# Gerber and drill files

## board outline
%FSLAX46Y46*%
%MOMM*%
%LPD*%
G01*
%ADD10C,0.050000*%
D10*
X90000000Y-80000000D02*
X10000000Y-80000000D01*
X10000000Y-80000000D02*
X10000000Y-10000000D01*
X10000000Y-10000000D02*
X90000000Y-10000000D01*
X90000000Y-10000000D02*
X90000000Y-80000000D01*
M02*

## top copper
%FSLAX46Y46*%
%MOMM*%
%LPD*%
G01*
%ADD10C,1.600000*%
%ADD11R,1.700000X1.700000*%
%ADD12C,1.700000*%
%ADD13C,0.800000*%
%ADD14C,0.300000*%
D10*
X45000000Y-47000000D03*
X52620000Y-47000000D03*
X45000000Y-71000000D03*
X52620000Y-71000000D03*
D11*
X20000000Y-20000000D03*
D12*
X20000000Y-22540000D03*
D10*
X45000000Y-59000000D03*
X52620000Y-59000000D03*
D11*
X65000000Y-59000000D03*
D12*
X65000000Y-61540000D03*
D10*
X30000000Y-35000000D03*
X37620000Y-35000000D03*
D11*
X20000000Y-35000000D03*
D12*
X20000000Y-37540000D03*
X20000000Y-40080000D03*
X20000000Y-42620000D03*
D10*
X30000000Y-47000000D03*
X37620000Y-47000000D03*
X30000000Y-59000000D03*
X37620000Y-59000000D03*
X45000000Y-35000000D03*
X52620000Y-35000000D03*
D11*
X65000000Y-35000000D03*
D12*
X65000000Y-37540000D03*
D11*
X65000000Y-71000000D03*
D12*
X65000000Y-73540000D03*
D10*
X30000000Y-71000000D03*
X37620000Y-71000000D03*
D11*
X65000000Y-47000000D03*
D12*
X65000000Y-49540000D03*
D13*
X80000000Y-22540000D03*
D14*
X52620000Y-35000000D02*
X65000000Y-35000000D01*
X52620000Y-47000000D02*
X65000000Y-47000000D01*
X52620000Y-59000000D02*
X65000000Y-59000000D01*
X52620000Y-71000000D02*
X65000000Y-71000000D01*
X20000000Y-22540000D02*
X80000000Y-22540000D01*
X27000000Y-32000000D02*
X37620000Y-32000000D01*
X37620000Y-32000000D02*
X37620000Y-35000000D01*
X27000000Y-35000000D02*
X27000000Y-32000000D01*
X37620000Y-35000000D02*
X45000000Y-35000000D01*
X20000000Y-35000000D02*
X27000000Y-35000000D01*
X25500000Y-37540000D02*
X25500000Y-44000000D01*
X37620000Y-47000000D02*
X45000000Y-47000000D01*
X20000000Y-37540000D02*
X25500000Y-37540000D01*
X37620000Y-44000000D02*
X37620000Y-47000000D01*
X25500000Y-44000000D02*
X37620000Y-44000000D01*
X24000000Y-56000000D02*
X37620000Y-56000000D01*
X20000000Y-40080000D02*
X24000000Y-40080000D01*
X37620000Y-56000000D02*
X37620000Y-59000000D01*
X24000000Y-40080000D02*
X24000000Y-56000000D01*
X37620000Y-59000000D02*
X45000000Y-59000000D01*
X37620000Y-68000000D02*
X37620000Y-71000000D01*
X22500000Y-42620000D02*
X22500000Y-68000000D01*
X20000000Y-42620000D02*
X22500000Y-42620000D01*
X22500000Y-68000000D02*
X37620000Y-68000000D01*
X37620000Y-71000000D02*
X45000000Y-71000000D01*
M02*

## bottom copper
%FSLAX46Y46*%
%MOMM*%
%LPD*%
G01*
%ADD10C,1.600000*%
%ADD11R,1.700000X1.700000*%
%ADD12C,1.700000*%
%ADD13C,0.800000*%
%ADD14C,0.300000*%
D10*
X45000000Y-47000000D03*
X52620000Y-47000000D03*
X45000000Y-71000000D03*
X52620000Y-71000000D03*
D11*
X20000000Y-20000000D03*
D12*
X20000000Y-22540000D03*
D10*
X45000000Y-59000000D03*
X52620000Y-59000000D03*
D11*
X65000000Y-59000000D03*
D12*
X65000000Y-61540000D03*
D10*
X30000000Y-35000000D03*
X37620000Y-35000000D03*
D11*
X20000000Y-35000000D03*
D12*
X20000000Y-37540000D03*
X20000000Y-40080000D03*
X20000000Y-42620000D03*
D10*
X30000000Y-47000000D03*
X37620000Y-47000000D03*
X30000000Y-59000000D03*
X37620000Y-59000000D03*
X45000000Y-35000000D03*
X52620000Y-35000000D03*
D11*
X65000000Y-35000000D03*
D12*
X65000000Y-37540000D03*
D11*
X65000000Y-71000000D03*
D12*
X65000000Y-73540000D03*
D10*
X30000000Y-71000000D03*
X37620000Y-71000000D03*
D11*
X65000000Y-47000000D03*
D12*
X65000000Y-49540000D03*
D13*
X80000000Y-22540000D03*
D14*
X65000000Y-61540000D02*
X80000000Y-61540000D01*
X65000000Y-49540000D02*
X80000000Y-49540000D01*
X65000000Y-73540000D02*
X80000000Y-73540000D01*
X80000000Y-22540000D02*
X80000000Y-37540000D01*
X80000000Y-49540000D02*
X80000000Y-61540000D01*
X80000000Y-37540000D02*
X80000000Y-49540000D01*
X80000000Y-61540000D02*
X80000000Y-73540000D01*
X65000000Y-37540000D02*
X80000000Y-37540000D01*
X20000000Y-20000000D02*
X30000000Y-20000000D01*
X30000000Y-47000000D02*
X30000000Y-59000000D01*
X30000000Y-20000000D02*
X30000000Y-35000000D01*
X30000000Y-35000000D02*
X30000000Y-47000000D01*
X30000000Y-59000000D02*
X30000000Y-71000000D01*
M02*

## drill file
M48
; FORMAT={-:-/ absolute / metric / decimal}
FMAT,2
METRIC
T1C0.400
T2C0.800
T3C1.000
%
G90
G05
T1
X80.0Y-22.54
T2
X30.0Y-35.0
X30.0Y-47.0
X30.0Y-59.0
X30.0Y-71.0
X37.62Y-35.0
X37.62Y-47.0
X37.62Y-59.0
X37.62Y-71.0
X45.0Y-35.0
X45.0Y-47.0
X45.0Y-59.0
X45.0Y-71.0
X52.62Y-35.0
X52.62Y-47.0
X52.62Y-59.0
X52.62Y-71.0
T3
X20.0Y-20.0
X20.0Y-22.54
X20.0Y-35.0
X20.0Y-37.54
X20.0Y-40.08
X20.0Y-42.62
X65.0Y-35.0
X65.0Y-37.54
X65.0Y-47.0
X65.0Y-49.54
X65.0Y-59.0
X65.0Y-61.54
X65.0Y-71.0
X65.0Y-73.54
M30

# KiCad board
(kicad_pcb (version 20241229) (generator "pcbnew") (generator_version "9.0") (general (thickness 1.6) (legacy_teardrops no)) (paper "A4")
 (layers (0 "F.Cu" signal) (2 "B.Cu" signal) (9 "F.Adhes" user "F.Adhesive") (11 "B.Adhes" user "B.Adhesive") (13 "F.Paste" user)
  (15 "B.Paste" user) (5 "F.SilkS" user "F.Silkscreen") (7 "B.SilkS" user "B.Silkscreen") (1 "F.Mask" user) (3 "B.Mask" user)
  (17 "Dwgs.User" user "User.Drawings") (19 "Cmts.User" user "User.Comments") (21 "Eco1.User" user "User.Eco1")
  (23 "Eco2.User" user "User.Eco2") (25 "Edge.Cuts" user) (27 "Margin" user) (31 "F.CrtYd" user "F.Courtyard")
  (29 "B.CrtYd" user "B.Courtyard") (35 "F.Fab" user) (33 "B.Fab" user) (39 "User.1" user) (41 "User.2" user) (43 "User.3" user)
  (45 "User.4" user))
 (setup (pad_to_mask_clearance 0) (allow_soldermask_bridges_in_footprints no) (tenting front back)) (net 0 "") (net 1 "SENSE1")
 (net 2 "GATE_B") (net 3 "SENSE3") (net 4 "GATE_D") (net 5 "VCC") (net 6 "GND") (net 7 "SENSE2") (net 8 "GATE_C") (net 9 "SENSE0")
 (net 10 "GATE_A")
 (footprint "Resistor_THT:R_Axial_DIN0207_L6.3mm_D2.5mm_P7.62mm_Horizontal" (layer "F.Cu") (at 45 47)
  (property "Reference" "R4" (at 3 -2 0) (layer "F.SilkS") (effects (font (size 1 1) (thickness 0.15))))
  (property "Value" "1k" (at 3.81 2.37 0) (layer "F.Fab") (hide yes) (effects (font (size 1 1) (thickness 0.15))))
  (pad "1" thru_hole circle (at 0 0) (size 1.6 1.6) (drill 0.8) (layers "*.Cu" "*.Mask") (remove_unused_layers no) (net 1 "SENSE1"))
  (pad "2" thru_hole circle (at 7.62 0) (size 1.6 1.6) (drill 0.8) (layers "*.Cu" "*.Mask") (remove_unused_layers no) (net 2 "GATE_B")))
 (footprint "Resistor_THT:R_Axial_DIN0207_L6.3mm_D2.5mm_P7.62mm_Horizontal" (layer "F.Cu") (at 45 71)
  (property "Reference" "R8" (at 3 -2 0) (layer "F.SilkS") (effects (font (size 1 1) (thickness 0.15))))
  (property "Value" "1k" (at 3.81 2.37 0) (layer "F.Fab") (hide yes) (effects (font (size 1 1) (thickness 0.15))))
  (pad "1" thru_hole circle (at 0 0) (size 1.6 1.6) (drill 0.8) (layers "*.Cu" "*.Mask") (remove_unused_layers no) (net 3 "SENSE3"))
  (pad "2" thru_hole circle (at 7.62 0) (size 1.6 1.6) (drill 0.8) (layers "*.Cu" "*.Mask") (remove_unused_layers no) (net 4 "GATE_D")))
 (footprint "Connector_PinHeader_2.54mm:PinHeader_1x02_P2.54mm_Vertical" (layer "F.Cu") (at 20 20)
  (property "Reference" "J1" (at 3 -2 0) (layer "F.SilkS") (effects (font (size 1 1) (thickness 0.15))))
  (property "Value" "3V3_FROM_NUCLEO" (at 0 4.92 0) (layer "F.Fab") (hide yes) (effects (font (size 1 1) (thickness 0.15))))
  (pad "1" thru_hole rect (at 0 0) (size 1.7 1.7) (drill 1) (layers "*.Cu" "*.Mask") (remove_unused_layers no) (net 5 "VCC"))
  (pad "2" thru_hole circle (at 0 2.54) (size 1.7 1.7) (drill 1) (layers "*.Cu" "*.Mask") (remove_unused_layers no) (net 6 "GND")))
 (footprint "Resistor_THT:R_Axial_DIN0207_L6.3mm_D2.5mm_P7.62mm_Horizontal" (layer "F.Cu") (at 45 59)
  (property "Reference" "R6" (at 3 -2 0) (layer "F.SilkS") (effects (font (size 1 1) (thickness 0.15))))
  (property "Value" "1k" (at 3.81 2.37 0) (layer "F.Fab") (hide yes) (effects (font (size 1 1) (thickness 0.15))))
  (pad "1" thru_hole circle (at 0 0) (size 1.6 1.6) (drill 0.8) (layers "*.Cu" "*.Mask") (remove_unused_layers no) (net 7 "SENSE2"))
  (pad "2" thru_hole circle (at 7.62 0) (size 1.6 1.6) (drill 0.8) (layers "*.Cu" "*.Mask") (remove_unused_layers no) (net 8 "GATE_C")))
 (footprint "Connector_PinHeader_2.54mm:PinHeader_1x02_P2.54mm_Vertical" (layer "F.Cu") (at 65 59)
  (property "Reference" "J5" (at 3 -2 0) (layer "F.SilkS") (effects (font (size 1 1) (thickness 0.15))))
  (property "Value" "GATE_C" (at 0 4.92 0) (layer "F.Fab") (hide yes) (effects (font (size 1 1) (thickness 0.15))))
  (pad "1" thru_hole rect (at 0 0) (size 1.7 1.7) (drill 1) (layers "*.Cu" "*.Mask") (remove_unused_layers no) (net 8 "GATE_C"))
  (pad "2" thru_hole circle (at 0 2.54) (size 1.7 1.7) (drill 1) (layers "*.Cu" "*.Mask") (remove_unused_layers no) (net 6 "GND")))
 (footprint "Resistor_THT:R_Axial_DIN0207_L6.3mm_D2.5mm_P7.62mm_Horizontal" (layer "F.Cu") (at 30 35)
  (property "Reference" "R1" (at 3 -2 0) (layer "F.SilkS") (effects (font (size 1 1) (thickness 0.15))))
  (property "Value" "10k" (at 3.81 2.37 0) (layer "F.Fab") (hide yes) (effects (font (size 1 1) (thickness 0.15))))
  (pad "1" thru_hole circle (at 0 0) (size 1.6 1.6) (drill 0.8) (layers "*.Cu" "*.Mask") (remove_unused_layers no) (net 5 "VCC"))
  (pad "2" thru_hole circle (at 7.62 0) (size 1.6 1.6) (drill 0.8) (layers "*.Cu" "*.Mask") (remove_unused_layers no) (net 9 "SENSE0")))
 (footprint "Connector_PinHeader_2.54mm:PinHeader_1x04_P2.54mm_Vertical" (layer "F.Cu") (at 20 35)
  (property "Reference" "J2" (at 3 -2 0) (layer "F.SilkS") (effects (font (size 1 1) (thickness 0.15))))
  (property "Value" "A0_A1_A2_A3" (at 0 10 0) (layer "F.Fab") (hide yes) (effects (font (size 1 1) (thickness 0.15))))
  (pad "1" thru_hole rect (at 0 0) (size 1.7 1.7) (drill 1) (layers "*.Cu" "*.Mask") (remove_unused_layers no) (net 9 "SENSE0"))
  (pad "2" thru_hole circle (at 0 2.54) (size 1.7 1.7) (drill 1) (layers "*.Cu" "*.Mask") (remove_unused_layers no) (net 1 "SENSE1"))
  (pad "3" thru_hole circle (at 0 5.08) (size 1.7 1.7) (drill 1) (layers "*.Cu" "*.Mask") (remove_unused_layers no) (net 7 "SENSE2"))
  (pad "4" thru_hole circle (at 0 7.62) (size 1.7 1.7) (drill 1) (layers "*.Cu" "*.Mask") (remove_unused_layers no) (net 3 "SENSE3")))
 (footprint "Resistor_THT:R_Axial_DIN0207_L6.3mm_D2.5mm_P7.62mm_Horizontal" (layer "F.Cu") (at 30 47)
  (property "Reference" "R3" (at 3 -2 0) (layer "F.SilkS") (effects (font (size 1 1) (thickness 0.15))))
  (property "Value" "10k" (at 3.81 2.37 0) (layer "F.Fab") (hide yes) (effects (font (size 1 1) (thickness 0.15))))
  (pad "1" thru_hole circle (at 0 0) (size 1.6 1.6) (drill 0.8) (layers "*.Cu" "*.Mask") (remove_unused_layers no) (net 5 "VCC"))
  (pad "2" thru_hole circle (at 7.62 0) (size 1.6 1.6) (drill 0.8) (layers "*.Cu" "*.Mask") (remove_unused_layers no) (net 1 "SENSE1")))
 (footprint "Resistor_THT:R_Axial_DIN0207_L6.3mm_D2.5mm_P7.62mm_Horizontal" (layer "F.Cu") (at 30 59)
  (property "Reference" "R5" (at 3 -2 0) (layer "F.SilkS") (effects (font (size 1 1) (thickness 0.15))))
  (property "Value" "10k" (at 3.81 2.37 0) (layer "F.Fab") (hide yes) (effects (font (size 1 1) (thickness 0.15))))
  (pad "1" thru_hole circle (at 0 0) (size 1.6 1.6) (drill 0.8) (layers "*.Cu" "*.Mask") (remove_unused_layers no) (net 5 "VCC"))
  (pad "2" thru_hole circle (at 7.62 0) (size 1.6 1.6) (drill 0.8) (layers "*.Cu" "*.Mask") (remove_unused_layers no) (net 7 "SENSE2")))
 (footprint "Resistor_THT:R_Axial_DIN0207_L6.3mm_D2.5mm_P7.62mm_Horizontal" (layer "F.Cu") (at 45 35)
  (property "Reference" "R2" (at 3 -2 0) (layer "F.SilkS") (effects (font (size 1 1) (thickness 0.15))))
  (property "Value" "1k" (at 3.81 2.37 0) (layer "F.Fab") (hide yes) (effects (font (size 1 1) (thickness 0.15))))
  (pad "1" thru_hole circle (at 0 0) (size 1.6 1.6) (drill 0.8) (layers "*.Cu" "*.Mask") (remove_unused_layers no) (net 9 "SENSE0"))
  (pad "2" thru_hole circle (at 7.62 0) (size 1.6 1.6) (drill 0.8) (layers "*.Cu" "*.Mask") (remove_unused_layers no) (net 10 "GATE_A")))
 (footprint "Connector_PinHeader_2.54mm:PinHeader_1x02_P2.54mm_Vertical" (layer "F.Cu") (at 65 35)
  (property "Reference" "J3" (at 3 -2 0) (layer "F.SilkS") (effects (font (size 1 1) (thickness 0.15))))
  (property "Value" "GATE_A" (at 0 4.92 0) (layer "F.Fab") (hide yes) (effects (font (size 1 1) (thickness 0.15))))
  (pad "1" thru_hole rect (at 0 0) (size 1.7 1.7) (drill 1) (layers "*.Cu" "*.Mask") (remove_unused_layers no) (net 10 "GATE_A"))
  (pad "2" thru_hole circle (at 0 2.54) (size 1.7 1.7) (drill 1) (layers "*.Cu" "*.Mask") (remove_unused_layers no) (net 6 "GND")))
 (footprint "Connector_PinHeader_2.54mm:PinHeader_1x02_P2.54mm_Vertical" (layer "F.Cu") (at 65 71)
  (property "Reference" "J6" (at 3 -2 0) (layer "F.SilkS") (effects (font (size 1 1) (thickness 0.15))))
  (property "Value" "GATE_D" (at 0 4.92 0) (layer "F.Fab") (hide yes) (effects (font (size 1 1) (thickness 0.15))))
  (pad "1" thru_hole rect (at 0 0) (size 1.7 1.7) (drill 1) (layers "*.Cu" "*.Mask") (remove_unused_layers no) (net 4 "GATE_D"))
  (pad "2" thru_hole circle (at 0 2.54) (size 1.7 1.7) (drill 1) (layers "*.Cu" "*.Mask") (remove_unused_layers no) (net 6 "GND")))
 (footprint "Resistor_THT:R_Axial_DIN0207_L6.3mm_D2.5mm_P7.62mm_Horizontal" (layer "F.Cu") (at 30 71)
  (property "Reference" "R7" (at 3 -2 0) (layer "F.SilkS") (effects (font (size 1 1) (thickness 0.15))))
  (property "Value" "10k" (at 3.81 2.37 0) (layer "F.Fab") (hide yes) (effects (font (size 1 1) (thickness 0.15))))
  (pad "1" thru_hole circle (at 0 0) (size 1.6 1.6) (drill 0.8) (layers "*.Cu" "*.Mask") (remove_unused_layers no) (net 5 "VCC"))
  (pad "2" thru_hole circle (at 7.62 0) (size 1.6 1.6) (drill 0.8) (layers "*.Cu" "*.Mask") (remove_unused_layers no) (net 3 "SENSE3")))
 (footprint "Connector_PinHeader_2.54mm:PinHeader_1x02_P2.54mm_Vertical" (layer "F.Cu") (at 65 47)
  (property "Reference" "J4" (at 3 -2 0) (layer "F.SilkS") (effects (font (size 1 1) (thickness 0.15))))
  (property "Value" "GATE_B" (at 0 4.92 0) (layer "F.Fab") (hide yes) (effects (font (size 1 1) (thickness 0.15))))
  (pad "1" thru_hole rect (at 0 0) (size 1.7 1.7) (drill 1) (layers "*.Cu" "*.Mask") (remove_unused_layers no) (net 2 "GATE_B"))
  (pad "2" thru_hole circle (at 0 2.54) (size 1.7 1.7) (drill 1) (layers "*.Cu" "*.Mask") (remove_unused_layers no) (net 6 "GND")))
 (gr_line (start 90 80) (end 10 80) (stroke (width 0.05) (type default)) (layer "Edge.Cuts"))
 (gr_line (start 10 80) (end 10 10) (stroke (width 0.05) (type default)) (layer "Edge.Cuts"))
 (gr_line (start 10 10) (end 90 10) (stroke (width 0.05) (type default)) (layer "Edge.Cuts"))
 (gr_line (start 90 10) (end 90 80) (stroke (width 0.05) (type default)) (layer "Edge.Cuts"))
 (segment (start 52.62 35) (end 65 35) (width 0.3) (layer "F.Cu") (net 10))
 (segment (start 52.62 47) (end 65 47) (width 0.3) (layer "F.Cu") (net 2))
 (segment (start 52.62 59) (end 65 59) (width 0.3) (layer "F.Cu") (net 8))
 (segment (start 52.62 71) (end 65 71) (width 0.3) (layer "F.Cu") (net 4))
 (segment (start 20 22.54) (end 80 22.54) (width 0.3) (layer "F.Cu") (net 6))
 (via (at 80 22.54) (size 0.8) (drill 0.4) (layers "F.Cu" "B.Cu") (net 6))
 (segment (start 65 61.54) (end 80 61.54) (width 0.3) (layer "B.Cu") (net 6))
 (segment (start 65 49.54) (end 80 49.54) (width 0.3) (layer "B.Cu") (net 6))
 (segment (start 65 73.54) (end 80 73.54) (width 0.3) (layer "B.Cu") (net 6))
 (segment (start 80 22.54) (end 80 37.54) (width 0.3) (layer "B.Cu") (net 6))
 (segment (start 80 49.54) (end 80 61.54) (width 0.3) (layer "B.Cu") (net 6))
 (segment (start 80 37.54) (end 80 49.54) (width 0.3) (layer "B.Cu") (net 6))
 (segment (start 80 61.54) (end 80 73.54) (width 0.3) (layer "B.Cu") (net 6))
 (segment (start 65 37.54) (end 80 37.54) (width 0.3) (layer "B.Cu") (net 6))
 (segment (start 27 32) (end 37.62 32) (width 0.3) (layer "F.Cu") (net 9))
 (segment (start 37.62 32) (end 37.62 35) (width 0.3) (layer "F.Cu") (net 9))
 (segment (start 27 35) (end 27 32) (width 0.3) (layer "F.Cu") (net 9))
 (segment (start 37.62 35) (end 45 35) (width 0.3) (layer "F.Cu") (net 9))
 (segment (start 20 35) (end 27 35) (width 0.3) (layer "F.Cu") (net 9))
 (segment (start 25.5 37.54) (end 25.5 44) (width 0.3) (layer "F.Cu") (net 1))
 (segment (start 37.62 47) (end 45 47) (width 0.3) (layer "F.Cu") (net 1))
 (segment (start 20 37.54) (end 25.5 37.54) (width 0.3) (layer "F.Cu") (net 1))
 (segment (start 37.62 44) (end 37.62 47) (width 0.3) (layer "F.Cu") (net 1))
 (segment (start 25.5 44) (end 37.62 44) (width 0.3) (layer "F.Cu") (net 1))
 (segment (start 24 56) (end 37.62 56) (width 0.3) (layer "F.Cu") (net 7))
 (segment (start 20 40.08) (end 24 40.08) (width 0.3) (layer "F.Cu") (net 7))
 (segment (start 37.62 56) (end 37.62 59) (width 0.3) (layer "F.Cu") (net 7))
 (segment (start 24 40.08) (end 24 56) (width 0.3) (layer "F.Cu") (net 7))
 (segment (start 37.62 59) (end 45 59) (width 0.3) (layer "F.Cu") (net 7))
 (segment (start 37.62 68) (end 37.62 71) (width 0.3) (layer "F.Cu") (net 3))
 (segment (start 22.5 42.62) (end 22.5 68) (width 0.3) (layer "F.Cu") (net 3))
 (segment (start 20 42.62) (end 22.5 42.62) (width 0.3) (layer "F.Cu") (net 3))
 (segment (start 22.5 68) (end 37.62 68) (width 0.3) (layer "F.Cu") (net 3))
 (segment (start 37.62 71) (end 45 71) (width 0.3) (layer "F.Cu") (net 3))
 (segment (start 20 20) (end 30 20) (width 0.3) (layer "B.Cu") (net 5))
 (segment (start 30 47) (end 30 59) (width 0.3) (layer "B.Cu") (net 5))
 (segment (start 30 20) (end 30 35) (width 0.3) (layer "B.Cu") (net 5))
 (segment (start 30 35) (end 30 47) (width 0.3) (layer "B.Cu") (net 5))
 (segment (start 30 59) (end 30 71) (width 0.3) (layer "B.Cu") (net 5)))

